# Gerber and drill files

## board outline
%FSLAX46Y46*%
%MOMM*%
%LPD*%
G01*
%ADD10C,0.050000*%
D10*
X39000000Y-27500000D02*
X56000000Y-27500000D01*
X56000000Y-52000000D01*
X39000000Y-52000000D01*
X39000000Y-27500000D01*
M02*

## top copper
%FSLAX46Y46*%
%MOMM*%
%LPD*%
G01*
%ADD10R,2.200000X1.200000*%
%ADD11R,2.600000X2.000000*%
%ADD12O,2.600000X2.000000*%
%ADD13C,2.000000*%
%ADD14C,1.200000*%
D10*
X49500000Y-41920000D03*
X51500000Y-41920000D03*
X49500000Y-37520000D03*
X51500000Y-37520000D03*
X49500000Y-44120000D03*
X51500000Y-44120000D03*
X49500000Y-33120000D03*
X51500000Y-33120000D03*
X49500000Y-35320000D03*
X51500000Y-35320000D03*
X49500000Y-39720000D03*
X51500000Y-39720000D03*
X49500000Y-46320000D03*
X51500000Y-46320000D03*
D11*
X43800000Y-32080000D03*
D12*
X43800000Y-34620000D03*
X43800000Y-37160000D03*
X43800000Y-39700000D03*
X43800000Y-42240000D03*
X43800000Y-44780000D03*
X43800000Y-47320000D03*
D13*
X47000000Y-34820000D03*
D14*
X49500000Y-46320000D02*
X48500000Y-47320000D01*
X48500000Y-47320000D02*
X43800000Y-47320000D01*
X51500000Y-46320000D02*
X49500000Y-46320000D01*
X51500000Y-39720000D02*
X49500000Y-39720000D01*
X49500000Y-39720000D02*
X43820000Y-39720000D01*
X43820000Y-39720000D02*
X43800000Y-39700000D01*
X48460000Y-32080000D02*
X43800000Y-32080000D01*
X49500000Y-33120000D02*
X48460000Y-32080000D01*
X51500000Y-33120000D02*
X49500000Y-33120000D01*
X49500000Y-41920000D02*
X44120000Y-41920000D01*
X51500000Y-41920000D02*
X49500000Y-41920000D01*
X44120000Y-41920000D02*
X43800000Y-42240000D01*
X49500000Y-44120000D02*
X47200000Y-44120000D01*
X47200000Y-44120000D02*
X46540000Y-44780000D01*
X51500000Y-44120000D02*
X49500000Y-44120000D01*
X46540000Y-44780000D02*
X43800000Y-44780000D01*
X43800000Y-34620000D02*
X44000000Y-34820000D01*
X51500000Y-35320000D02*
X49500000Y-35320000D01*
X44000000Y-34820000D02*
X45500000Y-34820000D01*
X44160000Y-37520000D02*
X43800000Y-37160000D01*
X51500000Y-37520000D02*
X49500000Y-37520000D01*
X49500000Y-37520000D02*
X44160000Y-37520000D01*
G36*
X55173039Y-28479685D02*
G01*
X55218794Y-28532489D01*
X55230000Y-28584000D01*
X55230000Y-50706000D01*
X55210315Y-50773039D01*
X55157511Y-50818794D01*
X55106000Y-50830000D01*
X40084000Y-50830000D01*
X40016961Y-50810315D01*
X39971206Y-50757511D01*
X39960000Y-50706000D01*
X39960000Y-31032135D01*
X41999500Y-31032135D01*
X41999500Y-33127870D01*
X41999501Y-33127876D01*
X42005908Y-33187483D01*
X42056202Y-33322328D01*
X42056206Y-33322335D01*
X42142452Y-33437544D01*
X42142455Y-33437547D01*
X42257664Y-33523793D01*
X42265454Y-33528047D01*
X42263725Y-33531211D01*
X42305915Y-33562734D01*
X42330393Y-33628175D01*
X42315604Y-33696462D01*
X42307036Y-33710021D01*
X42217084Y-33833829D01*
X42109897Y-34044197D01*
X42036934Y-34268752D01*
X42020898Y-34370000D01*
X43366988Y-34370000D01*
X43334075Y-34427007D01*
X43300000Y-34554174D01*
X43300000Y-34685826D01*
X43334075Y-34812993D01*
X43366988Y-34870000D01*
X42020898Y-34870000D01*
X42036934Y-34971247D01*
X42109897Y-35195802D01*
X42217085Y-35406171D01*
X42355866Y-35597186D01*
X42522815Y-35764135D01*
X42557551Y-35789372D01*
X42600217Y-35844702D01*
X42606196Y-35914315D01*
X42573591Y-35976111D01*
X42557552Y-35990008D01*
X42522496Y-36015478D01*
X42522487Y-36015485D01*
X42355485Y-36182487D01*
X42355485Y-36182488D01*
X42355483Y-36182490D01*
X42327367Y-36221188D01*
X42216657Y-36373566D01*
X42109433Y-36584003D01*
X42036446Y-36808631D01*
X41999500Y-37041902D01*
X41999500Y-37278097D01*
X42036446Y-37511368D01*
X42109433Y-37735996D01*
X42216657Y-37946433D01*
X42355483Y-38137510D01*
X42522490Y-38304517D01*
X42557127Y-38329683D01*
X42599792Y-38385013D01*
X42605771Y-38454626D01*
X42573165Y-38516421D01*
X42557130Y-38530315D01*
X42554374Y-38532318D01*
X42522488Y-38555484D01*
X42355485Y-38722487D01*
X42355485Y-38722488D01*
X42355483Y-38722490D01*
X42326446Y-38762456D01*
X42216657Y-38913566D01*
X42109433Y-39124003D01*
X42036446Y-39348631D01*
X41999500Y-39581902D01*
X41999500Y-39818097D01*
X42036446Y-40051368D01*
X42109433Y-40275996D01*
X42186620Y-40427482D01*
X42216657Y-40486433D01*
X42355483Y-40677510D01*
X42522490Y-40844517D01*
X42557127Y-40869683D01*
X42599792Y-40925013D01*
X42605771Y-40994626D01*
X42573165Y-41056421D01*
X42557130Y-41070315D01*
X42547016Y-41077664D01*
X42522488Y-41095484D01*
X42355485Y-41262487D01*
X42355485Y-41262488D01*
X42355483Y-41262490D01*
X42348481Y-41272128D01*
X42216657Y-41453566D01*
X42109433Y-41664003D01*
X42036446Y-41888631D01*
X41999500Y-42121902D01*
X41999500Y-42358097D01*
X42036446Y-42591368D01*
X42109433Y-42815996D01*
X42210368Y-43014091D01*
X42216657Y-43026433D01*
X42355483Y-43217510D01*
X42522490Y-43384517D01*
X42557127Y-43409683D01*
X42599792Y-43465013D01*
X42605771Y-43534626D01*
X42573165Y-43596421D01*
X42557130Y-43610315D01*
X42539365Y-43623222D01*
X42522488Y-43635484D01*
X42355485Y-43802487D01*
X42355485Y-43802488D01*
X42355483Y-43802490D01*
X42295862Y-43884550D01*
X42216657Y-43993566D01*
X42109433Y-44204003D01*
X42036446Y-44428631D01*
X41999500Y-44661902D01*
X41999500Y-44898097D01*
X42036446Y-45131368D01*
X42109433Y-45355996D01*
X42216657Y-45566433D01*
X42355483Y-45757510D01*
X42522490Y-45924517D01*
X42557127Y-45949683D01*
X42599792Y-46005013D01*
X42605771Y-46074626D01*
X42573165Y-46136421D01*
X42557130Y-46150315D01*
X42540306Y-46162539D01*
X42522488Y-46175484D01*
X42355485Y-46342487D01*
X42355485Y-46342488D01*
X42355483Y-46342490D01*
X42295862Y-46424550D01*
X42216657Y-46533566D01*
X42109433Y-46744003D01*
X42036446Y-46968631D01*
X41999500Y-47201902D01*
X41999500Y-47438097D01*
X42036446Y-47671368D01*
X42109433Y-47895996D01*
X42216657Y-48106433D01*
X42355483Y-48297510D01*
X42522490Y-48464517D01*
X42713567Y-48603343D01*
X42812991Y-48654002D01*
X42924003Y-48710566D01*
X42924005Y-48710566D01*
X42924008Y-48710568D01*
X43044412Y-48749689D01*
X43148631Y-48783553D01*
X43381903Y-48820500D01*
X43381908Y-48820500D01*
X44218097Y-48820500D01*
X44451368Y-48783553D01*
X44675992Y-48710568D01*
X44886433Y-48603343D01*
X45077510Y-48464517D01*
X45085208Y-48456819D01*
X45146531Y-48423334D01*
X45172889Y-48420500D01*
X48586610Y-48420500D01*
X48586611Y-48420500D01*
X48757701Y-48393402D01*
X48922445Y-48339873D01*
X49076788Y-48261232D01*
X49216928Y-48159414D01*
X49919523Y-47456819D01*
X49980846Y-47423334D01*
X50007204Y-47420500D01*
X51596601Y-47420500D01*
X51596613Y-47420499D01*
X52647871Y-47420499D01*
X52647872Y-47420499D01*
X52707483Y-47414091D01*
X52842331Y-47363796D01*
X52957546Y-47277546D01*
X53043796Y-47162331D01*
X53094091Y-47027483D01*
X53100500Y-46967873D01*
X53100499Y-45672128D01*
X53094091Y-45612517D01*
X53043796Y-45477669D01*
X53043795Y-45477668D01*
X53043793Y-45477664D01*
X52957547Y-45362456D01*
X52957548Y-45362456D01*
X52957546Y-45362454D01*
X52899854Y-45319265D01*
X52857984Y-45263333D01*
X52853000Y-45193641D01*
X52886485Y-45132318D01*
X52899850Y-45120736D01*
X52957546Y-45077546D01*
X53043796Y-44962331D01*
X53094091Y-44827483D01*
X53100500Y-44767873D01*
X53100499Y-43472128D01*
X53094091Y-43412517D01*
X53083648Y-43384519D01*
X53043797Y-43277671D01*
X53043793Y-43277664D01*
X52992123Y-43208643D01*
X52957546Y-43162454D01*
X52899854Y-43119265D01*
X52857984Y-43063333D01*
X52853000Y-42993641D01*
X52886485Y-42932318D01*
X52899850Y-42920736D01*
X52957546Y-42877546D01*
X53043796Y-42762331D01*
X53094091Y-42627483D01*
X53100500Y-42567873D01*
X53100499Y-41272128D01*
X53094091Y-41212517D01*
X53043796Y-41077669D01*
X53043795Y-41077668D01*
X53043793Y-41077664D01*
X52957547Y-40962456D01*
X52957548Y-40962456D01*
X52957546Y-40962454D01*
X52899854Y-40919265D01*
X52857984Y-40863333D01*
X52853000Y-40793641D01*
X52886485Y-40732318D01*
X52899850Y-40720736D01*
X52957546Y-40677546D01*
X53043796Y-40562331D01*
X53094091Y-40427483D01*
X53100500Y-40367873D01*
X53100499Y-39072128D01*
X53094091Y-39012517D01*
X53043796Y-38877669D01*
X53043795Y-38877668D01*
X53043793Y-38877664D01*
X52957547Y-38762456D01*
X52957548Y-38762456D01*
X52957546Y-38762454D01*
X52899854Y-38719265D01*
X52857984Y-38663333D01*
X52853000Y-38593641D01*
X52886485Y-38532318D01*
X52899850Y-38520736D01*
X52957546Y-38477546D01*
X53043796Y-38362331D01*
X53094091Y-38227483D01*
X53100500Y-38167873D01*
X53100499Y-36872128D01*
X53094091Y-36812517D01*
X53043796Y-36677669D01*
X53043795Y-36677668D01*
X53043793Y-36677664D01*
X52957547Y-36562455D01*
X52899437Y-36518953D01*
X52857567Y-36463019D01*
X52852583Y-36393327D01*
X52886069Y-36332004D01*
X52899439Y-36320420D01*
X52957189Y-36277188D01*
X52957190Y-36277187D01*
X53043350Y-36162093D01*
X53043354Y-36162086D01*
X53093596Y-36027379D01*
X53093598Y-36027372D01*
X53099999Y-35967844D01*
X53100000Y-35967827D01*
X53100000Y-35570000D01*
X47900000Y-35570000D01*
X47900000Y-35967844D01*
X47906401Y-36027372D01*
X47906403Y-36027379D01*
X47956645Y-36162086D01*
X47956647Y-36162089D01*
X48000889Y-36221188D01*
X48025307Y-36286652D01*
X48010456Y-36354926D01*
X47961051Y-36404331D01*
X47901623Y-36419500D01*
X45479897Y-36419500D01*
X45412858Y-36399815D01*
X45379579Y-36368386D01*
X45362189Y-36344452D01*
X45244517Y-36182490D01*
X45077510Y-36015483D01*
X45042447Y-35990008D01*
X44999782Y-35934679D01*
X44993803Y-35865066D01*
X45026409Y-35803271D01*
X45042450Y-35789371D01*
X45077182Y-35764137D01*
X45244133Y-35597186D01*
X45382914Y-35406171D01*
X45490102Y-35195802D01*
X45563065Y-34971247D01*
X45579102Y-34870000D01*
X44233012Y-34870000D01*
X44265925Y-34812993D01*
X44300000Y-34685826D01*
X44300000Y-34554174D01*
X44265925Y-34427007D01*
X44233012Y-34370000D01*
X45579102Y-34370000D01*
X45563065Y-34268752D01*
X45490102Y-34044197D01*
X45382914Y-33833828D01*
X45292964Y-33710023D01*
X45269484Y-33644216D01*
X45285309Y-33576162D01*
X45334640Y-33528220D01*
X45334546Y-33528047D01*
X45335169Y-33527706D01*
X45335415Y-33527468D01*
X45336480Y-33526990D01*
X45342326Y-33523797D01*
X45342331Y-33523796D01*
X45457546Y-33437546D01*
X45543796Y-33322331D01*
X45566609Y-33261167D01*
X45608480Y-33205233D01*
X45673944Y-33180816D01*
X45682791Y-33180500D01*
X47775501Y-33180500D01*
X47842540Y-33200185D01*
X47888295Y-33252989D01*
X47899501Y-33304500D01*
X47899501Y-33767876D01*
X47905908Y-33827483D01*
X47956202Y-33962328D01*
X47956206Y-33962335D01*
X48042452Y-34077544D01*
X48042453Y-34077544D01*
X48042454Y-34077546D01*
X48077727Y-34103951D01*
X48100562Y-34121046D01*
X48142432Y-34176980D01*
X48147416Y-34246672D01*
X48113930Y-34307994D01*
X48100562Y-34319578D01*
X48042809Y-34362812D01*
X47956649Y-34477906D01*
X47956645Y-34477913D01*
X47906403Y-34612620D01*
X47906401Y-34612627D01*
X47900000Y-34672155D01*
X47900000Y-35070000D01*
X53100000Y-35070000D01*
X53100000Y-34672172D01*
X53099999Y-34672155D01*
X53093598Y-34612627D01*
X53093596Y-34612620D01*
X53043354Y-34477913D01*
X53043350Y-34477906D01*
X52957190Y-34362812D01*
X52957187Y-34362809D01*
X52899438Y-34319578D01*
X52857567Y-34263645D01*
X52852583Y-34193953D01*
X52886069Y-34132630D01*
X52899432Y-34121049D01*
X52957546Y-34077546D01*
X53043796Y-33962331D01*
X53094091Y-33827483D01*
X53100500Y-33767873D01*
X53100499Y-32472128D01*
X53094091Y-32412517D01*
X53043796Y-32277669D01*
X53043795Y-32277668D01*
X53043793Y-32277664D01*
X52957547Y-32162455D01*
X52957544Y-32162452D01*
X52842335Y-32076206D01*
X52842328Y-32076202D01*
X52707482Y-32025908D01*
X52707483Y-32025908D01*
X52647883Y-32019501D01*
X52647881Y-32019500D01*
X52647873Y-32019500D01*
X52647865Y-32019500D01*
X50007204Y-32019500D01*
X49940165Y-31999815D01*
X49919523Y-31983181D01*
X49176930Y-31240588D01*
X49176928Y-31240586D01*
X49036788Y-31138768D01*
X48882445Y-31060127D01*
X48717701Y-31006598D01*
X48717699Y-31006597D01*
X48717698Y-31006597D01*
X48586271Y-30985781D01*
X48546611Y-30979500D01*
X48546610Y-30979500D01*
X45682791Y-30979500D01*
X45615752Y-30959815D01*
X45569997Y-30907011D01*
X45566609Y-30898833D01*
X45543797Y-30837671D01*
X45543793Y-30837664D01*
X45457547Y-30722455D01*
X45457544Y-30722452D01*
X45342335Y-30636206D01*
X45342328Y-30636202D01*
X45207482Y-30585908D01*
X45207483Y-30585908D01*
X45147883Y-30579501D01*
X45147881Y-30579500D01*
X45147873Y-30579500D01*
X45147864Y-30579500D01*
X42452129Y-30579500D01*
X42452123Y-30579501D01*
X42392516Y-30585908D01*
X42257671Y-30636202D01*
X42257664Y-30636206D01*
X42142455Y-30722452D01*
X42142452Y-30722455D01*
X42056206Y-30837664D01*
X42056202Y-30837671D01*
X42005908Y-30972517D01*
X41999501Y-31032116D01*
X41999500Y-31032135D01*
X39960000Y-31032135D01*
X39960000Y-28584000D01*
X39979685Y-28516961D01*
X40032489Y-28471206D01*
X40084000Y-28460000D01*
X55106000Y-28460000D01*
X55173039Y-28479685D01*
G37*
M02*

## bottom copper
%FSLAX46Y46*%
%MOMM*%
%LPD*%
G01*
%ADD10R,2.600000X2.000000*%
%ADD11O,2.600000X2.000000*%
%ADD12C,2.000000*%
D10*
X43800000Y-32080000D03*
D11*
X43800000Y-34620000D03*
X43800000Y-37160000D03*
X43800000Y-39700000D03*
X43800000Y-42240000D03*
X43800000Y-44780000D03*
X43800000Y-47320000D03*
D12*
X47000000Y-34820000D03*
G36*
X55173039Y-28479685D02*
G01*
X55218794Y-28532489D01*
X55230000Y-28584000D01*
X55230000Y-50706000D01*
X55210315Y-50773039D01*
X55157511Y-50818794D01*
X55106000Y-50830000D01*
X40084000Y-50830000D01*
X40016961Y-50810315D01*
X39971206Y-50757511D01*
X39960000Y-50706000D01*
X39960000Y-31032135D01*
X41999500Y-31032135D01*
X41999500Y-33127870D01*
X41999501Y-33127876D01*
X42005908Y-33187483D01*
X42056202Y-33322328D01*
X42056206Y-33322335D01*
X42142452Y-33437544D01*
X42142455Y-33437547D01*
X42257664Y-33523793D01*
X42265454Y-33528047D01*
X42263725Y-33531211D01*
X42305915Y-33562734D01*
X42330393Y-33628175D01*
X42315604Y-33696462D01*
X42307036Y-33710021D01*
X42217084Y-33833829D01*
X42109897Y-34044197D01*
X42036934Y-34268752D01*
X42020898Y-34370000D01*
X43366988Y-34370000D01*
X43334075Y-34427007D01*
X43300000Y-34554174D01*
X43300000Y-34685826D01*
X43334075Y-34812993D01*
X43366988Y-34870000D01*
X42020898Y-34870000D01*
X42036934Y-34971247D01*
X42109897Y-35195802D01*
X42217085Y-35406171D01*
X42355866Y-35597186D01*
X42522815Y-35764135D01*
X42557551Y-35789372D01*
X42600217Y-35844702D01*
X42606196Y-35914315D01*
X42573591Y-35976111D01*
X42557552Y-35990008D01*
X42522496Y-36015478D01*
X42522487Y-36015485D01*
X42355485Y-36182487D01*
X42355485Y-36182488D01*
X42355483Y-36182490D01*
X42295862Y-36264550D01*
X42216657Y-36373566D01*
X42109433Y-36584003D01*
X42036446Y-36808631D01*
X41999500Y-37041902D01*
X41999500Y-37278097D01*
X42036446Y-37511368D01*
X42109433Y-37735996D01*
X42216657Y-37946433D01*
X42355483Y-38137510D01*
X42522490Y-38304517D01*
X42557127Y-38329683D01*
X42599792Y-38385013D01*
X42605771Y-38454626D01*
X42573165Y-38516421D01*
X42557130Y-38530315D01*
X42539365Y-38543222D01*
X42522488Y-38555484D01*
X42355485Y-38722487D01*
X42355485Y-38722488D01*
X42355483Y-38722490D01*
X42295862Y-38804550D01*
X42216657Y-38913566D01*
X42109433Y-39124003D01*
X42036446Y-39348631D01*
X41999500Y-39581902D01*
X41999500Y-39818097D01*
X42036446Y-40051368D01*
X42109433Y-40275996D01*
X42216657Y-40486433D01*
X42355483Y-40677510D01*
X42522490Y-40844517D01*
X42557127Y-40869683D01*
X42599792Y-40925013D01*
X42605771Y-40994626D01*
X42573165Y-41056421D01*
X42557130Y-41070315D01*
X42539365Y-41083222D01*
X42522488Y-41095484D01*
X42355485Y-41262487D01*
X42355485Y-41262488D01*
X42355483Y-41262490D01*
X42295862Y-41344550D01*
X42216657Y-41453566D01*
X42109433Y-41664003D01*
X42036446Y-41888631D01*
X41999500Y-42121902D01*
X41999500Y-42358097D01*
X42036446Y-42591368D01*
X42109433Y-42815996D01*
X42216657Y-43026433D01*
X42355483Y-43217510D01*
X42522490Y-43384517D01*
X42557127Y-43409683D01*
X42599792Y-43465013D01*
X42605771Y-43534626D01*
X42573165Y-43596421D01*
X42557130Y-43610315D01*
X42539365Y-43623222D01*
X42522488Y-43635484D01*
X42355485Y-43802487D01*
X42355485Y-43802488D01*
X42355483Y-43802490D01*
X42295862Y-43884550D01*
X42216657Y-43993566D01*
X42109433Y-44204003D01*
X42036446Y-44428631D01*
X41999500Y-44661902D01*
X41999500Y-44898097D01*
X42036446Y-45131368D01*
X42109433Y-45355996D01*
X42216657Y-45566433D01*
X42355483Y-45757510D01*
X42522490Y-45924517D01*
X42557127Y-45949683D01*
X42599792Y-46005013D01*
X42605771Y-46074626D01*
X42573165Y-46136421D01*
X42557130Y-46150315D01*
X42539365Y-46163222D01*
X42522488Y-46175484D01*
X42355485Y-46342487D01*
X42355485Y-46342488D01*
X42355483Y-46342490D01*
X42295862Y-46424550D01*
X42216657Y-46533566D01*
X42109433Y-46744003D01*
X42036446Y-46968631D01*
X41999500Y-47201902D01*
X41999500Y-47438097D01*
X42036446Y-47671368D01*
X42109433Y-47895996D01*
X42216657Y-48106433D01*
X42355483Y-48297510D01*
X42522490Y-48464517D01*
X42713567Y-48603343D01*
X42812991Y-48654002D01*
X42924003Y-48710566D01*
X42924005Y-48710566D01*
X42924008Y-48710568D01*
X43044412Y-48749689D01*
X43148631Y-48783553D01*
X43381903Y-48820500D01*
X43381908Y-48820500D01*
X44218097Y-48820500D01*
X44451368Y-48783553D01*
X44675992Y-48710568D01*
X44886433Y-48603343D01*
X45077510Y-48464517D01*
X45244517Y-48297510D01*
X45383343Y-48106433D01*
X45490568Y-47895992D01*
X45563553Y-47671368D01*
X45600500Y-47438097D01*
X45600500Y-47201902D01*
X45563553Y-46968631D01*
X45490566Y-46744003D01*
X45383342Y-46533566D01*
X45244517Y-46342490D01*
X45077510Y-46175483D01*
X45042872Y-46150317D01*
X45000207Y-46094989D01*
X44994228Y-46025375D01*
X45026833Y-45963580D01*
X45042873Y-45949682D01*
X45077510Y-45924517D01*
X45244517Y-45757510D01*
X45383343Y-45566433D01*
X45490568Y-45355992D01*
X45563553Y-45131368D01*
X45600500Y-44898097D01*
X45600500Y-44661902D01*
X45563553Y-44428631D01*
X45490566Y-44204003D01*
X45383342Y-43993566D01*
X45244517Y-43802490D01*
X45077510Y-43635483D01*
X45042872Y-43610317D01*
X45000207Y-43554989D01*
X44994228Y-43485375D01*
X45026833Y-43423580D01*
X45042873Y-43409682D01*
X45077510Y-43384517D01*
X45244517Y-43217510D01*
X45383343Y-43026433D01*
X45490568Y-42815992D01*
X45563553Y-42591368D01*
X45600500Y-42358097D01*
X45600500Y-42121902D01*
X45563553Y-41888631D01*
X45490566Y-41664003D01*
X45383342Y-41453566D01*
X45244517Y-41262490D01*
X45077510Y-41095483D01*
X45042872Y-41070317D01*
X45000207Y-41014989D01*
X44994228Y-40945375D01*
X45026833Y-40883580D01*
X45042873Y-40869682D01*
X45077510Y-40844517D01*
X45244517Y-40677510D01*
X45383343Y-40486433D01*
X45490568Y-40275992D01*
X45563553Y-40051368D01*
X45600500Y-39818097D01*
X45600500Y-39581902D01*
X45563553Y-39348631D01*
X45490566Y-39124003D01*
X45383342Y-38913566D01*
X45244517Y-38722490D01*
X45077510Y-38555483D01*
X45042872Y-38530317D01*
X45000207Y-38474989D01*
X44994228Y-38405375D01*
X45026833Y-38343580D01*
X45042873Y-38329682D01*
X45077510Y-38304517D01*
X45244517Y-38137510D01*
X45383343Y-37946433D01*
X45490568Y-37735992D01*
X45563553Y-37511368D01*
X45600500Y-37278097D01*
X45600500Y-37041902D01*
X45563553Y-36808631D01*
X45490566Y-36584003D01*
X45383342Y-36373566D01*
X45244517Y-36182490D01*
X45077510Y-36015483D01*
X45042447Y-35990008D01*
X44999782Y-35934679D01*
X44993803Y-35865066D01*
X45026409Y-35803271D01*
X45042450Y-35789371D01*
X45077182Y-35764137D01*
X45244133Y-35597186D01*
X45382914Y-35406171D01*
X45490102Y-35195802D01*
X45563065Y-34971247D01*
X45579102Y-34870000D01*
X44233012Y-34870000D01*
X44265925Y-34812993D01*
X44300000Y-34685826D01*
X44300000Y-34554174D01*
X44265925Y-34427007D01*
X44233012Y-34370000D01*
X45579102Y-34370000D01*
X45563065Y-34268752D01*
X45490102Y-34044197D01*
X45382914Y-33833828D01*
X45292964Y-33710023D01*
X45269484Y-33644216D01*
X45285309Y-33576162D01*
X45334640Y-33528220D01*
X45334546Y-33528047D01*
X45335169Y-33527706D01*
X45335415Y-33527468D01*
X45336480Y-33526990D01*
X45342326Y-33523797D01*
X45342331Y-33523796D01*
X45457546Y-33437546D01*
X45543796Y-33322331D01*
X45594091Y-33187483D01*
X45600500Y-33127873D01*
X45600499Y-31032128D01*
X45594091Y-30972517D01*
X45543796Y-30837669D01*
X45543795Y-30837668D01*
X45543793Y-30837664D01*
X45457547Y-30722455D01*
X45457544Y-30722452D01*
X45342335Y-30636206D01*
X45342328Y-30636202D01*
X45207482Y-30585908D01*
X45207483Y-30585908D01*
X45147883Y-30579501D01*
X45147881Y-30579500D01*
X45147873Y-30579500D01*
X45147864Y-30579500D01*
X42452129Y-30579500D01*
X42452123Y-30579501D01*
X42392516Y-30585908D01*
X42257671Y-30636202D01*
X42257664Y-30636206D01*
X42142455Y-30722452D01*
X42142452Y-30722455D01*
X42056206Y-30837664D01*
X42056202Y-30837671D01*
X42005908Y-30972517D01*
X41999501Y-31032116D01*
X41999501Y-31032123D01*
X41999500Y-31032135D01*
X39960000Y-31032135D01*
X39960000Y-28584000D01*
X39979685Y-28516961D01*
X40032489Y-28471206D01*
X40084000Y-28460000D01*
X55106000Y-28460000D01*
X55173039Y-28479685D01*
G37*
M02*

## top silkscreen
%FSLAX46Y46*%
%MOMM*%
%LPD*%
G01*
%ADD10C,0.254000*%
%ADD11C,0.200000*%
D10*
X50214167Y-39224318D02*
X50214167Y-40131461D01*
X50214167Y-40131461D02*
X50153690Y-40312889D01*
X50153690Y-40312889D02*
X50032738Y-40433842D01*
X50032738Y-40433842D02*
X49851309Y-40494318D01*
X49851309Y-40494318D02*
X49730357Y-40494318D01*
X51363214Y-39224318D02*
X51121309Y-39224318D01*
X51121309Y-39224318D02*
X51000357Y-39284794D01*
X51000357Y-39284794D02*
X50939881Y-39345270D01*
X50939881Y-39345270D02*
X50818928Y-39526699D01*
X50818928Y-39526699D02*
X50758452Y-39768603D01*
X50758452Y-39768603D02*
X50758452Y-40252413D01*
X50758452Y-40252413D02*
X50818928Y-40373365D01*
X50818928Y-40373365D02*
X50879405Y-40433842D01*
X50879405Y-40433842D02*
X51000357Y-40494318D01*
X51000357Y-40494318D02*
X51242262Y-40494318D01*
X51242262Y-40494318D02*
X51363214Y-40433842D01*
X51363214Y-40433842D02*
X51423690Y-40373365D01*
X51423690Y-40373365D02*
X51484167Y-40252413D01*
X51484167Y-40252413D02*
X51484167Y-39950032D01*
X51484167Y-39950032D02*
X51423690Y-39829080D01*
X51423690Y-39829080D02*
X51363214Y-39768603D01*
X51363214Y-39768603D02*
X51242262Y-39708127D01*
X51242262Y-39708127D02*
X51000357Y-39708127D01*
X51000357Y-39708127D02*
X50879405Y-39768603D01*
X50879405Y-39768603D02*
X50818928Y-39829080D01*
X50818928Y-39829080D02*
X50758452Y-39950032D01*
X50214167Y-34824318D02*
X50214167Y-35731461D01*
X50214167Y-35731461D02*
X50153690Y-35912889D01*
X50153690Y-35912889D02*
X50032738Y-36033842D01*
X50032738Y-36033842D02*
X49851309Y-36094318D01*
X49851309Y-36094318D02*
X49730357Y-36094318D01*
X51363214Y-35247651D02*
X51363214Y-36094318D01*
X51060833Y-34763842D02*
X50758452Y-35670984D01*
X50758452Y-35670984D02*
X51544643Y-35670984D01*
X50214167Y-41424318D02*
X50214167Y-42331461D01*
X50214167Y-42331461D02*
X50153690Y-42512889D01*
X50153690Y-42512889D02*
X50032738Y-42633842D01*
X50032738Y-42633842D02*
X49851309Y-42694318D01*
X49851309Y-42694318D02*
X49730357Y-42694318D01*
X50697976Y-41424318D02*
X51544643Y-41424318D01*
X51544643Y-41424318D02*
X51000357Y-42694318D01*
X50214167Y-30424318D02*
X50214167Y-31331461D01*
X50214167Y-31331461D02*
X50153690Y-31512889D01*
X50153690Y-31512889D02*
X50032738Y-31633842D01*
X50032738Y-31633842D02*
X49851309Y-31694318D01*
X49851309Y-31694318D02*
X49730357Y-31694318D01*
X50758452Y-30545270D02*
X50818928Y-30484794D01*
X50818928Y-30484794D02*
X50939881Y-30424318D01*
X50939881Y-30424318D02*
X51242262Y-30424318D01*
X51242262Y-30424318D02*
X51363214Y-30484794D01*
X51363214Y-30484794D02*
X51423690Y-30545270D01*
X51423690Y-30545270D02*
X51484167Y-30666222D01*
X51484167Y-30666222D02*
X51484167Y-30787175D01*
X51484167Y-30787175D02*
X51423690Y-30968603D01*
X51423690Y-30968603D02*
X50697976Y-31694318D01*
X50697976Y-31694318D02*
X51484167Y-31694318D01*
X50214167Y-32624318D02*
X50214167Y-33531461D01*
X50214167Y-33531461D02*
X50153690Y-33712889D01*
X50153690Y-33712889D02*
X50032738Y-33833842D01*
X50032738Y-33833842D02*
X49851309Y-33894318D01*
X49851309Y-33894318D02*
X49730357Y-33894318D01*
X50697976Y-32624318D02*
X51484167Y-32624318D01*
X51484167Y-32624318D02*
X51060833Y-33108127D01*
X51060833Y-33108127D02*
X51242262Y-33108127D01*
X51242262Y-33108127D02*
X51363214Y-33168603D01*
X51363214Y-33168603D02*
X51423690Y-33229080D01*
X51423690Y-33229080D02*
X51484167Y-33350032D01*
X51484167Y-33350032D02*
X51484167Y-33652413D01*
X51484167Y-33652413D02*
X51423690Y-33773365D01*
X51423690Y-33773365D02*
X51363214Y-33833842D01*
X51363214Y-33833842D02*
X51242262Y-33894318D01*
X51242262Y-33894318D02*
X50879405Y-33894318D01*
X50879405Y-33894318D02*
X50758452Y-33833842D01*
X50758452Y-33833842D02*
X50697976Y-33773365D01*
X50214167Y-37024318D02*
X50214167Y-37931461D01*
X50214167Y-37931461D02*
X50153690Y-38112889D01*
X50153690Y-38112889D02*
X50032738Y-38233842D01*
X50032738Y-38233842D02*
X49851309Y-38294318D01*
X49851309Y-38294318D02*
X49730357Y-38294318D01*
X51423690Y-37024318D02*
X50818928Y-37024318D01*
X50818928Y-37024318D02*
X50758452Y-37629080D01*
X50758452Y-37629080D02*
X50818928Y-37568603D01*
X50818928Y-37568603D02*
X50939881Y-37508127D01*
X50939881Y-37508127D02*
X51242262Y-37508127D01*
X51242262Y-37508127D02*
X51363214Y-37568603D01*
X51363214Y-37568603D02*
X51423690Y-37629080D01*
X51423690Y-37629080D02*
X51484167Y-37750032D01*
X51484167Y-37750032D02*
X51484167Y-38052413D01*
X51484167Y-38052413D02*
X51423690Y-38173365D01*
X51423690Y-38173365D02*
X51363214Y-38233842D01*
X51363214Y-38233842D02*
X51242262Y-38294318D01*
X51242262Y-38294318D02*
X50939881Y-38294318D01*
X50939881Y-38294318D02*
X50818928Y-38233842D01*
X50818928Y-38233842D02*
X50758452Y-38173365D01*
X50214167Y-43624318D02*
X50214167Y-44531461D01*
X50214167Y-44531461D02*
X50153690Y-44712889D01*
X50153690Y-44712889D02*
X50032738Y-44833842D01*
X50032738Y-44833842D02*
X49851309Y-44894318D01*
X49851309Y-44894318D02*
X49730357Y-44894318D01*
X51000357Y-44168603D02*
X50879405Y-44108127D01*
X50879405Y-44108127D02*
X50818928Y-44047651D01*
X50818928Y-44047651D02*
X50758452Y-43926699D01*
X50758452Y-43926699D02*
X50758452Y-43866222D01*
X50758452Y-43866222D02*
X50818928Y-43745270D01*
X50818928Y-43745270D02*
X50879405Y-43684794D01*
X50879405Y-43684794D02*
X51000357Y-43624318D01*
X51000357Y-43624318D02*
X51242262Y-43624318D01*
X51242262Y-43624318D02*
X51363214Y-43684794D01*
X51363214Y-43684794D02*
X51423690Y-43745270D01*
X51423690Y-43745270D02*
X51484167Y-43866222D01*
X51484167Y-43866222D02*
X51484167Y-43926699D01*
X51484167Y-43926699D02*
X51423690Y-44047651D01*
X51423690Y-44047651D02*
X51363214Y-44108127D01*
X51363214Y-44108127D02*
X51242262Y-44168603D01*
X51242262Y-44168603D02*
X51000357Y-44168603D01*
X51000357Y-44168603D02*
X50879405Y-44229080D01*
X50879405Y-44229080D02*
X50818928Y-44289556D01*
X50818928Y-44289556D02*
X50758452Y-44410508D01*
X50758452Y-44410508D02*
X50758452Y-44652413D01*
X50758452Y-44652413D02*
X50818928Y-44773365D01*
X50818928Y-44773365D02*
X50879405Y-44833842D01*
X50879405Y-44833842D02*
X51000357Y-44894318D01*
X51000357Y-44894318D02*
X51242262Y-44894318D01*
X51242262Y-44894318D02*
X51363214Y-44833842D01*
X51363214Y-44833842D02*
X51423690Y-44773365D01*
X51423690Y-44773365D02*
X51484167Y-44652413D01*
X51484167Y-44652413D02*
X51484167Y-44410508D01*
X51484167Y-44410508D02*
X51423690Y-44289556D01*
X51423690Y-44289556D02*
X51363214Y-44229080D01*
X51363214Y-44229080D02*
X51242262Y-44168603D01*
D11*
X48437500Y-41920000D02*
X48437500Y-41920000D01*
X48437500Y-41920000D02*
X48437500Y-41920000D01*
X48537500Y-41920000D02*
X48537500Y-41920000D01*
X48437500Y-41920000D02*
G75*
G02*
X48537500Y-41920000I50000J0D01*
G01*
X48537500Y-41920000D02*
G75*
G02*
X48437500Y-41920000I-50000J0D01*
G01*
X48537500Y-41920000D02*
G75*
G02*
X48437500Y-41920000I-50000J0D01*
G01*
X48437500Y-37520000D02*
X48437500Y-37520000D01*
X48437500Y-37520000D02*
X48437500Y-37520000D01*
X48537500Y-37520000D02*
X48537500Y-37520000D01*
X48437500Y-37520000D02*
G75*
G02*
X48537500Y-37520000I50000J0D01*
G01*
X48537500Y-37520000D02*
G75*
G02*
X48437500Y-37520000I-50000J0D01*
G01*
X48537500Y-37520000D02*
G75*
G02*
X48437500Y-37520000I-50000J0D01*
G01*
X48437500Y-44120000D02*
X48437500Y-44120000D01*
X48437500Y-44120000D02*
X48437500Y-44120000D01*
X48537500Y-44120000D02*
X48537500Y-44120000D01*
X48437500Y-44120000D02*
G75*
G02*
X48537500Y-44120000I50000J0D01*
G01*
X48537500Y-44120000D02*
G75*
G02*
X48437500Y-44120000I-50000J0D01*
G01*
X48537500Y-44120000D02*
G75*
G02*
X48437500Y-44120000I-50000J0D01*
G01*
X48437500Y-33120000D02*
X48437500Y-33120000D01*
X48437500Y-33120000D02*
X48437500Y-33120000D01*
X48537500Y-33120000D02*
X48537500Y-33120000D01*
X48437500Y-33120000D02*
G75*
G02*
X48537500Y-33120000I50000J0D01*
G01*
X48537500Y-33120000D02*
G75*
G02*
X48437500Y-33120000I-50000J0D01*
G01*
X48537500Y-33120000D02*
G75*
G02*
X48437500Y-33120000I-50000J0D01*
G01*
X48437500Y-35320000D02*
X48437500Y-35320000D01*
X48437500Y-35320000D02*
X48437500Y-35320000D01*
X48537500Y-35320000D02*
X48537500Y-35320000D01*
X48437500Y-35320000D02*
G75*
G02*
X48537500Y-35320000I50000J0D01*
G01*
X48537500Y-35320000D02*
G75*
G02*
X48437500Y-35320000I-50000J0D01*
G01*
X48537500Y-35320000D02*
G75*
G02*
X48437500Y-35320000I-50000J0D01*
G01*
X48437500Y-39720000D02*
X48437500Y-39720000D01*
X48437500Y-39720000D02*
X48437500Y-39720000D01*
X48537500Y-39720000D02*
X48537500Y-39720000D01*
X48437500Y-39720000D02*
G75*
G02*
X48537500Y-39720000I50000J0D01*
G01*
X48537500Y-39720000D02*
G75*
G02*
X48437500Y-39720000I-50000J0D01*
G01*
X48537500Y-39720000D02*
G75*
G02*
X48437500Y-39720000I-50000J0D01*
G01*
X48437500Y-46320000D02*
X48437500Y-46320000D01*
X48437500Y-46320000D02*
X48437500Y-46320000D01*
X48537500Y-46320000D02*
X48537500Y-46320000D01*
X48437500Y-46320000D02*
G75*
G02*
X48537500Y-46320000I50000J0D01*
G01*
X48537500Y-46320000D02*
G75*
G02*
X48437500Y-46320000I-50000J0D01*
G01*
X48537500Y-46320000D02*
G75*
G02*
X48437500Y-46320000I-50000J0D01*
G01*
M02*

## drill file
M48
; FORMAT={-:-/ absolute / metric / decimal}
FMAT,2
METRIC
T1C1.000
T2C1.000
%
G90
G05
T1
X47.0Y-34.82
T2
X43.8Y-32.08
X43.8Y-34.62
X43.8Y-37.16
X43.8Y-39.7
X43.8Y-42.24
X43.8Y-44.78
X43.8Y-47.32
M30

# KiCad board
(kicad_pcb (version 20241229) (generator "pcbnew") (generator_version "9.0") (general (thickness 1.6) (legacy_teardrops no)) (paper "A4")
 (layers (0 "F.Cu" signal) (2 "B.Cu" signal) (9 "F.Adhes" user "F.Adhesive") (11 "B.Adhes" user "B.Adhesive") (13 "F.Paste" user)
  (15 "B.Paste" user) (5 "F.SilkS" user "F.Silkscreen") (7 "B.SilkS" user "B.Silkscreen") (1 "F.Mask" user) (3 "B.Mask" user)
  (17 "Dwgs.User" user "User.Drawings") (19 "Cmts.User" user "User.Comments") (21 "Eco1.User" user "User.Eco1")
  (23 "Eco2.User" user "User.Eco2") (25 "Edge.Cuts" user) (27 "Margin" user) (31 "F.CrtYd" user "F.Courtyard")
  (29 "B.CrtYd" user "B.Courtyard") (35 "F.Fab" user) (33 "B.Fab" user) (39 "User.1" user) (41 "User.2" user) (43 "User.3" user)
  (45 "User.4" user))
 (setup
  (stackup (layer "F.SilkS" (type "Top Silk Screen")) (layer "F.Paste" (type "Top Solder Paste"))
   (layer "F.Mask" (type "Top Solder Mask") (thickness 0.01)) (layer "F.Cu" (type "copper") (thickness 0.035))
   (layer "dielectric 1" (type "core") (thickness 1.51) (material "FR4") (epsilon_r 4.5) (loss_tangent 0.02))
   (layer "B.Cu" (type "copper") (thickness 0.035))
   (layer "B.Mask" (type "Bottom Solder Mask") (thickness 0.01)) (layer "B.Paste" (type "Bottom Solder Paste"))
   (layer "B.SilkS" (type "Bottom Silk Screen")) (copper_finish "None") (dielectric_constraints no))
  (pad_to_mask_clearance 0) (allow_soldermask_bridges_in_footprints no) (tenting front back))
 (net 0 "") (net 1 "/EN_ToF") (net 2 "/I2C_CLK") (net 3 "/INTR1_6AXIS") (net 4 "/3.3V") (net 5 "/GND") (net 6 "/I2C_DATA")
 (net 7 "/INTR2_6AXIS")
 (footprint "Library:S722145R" (layer "F.Cu") (at 50.6375 41.92)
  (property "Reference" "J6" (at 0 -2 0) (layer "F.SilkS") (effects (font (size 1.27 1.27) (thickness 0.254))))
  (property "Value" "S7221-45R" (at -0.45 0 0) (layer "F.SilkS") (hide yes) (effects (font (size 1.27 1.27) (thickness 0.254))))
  (fp_line (start -2.2 0) (end -2.2 0) (stroke (width 0.2) (type solid)) (layer "F.SilkS"))
  (fp_line (start -2.2 0) (end -2.2 0) (stroke (width 0.2) (type solid)) (layer "F.SilkS"))
  (fp_line (start -2.1 0) (end -2.1 0) (stroke (width 0.2) (type solid)) (layer "F.SilkS"))
  (fp_arc (start -2.2 0) (mid -2.15 -0.05) (end -2.1 0) (stroke (width 0.2) (type solid)) (layer "F.SilkS"))
  (fp_arc (start -2.1 0) (mid -2.15 0.05) (end -2.2 0) (stroke (width 0.2) (type solid)) (layer "F.SilkS"))
  (fp_arc (start -2.1 0) (mid -2.15 0.05) (end -2.2 0) (stroke (width 0.2) (type solid)) (layer "F.SilkS"))
  (pad "1" smd rect (at -1.1375 0) (size 2.2 1.2) (layers "F.Cu" "F.Mask" "F.Paste") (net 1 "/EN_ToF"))
  (pad "2" smd rect (at 0.8625 0) (size 2.2 1.2) (layers "F.Cu" "F.Mask" "F.Paste") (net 1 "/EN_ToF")))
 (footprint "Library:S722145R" (layer "F.Cu") (at 50.6375 37.52)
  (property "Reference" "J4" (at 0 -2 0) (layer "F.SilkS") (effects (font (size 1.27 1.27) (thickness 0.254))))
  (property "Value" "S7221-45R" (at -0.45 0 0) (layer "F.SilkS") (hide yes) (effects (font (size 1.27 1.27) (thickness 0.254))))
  (fp_line (start -2.2 0) (end -2.2 0) (stroke (width 0.2) (type solid)) (layer "F.SilkS"))
  (fp_line (start -2.2 0) (end -2.2 0) (stroke (width 0.2) (type solid)) (layer "F.SilkS"))
  (fp_line (start -2.1 0) (end -2.1 0) (stroke (width 0.2) (type solid)) (layer "F.SilkS"))
  (fp_arc (start -2.2 0) (mid -2.15 -0.05) (end -2.1 0) (stroke (width 0.2) (type solid)) (layer "F.SilkS"))
  (fp_arc (start -2.1 0) (mid -2.15 0.05) (end -2.2 0) (stroke (width 0.2) (type solid)) (layer "F.SilkS"))
  (fp_arc (start -2.1 0) (mid -2.15 0.05) (end -2.2 0) (stroke (width 0.2) (type solid)) (layer "F.SilkS"))
  (pad "1" smd rect (at -1.1375 0) (size 2.2 1.2) (layers "F.Cu" "F.Mask" "F.Paste") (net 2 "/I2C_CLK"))
  (pad "2" smd rect (at 0.8625 0) (size 2.2 1.2) (layers "F.Cu" "F.Mask" "F.Paste") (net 2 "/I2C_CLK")))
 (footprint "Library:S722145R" (layer "F.Cu") (at 50.6375 44.12)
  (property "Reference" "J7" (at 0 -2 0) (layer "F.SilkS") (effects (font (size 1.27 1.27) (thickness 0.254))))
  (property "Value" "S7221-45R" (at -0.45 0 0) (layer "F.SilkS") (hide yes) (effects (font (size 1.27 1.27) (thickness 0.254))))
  (fp_line (start -2.2 0) (end -2.2 0) (stroke (width 0.2) (type solid)) (layer "F.SilkS"))
  (fp_line (start -2.2 0) (end -2.2 0) (stroke (width 0.2) (type solid)) (layer "F.SilkS"))
  (fp_line (start -2.1 0) (end -2.1 0) (stroke (width 0.2) (type solid)) (layer "F.SilkS"))
  (fp_arc (start -2.2 0) (mid -2.15 -0.05) (end -2.1 0) (stroke (width 0.2) (type solid)) (layer "F.SilkS"))
  (fp_arc (start -2.1 0) (mid -2.15 0.05) (end -2.2 0) (stroke (width 0.2) (type solid)) (layer "F.SilkS"))
  (fp_arc (start -2.1 0) (mid -2.15 0.05) (end -2.2 0) (stroke (width 0.2) (type solid)) (layer "F.SilkS"))
  (pad "1" smd rect (at -1.1375 0) (size 2.2 1.2) (layers "F.Cu" "F.Mask" "F.Paste") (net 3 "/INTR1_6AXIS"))
  (pad "2" smd rect (at 0.8625 0) (size 2.2 1.2) (layers "F.Cu" "F.Mask" "F.Paste") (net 3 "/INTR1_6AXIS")))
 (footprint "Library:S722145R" (layer "F.Cu") (at 50.6375 33.12)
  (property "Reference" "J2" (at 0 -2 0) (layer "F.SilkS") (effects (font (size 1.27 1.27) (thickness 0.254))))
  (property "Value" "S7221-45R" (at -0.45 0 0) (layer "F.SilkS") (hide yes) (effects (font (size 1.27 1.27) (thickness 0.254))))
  (fp_line (start -2.2 0) (end -2.2 0) (stroke (width 0.2) (type solid)) (layer "F.SilkS"))
  (fp_line (start -2.2 0) (end -2.2 0) (stroke (width 0.2) (type solid)) (layer "F.SilkS"))
  (fp_line (start -2.1 0) (end -2.1 0) (stroke (width 0.2) (type solid)) (layer "F.SilkS"))
  (fp_arc (start -2.2 0) (mid -2.15 -0.05) (end -2.1 0) (stroke (width 0.2) (type solid)) (layer "F.SilkS"))
  (fp_arc (start -2.1 0) (mid -2.15 0.05) (end -2.2 0) (stroke (width 0.2) (type solid)) (layer "F.SilkS"))
  (fp_arc (start -2.1 0) (mid -2.15 0.05) (end -2.2 0) (stroke (width 0.2) (type solid)) (layer "F.SilkS"))
  (pad "1" smd rect (at -1.1375 0) (size 2.2 1.2) (layers "F.Cu" "F.Mask" "F.Paste") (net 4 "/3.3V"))
  (pad "2" smd rect (at 0.8625 0) (size 2.2 1.2) (layers "F.Cu" "F.Mask" "F.Paste") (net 4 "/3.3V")))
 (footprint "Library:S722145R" (layer "F.Cu") (at 50.6375 35.32)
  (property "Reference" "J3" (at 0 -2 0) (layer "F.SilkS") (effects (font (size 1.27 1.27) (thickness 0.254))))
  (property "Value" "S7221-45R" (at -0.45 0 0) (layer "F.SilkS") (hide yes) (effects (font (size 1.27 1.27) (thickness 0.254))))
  (fp_line (start -2.2 0) (end -2.2 0) (stroke (width 0.2) (type solid)) (layer "F.SilkS"))
  (fp_line (start -2.2 0) (end -2.2 0) (stroke (width 0.2) (type solid)) (layer "F.SilkS"))
  (fp_line (start -2.1 0) (end -2.1 0) (stroke (width 0.2) (type solid)) (layer "F.SilkS"))
  (fp_arc (start -2.2 0) (mid -2.15 -0.05) (end -2.1 0) (stroke (width 0.2) (type solid)) (layer "F.SilkS"))
  (fp_arc (start -2.1 0) (mid -2.15 0.05) (end -2.2 0) (stroke (width 0.2) (type solid)) (layer "F.SilkS"))
  (fp_arc (start -2.1 0) (mid -2.15 0.05) (end -2.2 0) (stroke (width 0.2) (type solid)) (layer "F.SilkS"))
  (pad "1" smd rect (at -1.1375 0) (size 2.2 1.2) (layers "F.Cu" "F.Mask" "F.Paste") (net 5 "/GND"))
  (pad "2" smd rect (at 0.8625 0) (size 2.2 1.2) (layers "F.Cu" "F.Mask" "F.Paste") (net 5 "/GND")))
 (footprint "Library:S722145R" (layer "F.Cu") (at 50.6375 39.72)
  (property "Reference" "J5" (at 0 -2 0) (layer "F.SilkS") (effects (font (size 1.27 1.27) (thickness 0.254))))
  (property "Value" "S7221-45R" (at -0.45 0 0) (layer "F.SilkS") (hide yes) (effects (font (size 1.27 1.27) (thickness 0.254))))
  (fp_line (start -2.2 0) (end -2.2 0) (stroke (width 0.2) (type solid)) (layer "F.SilkS"))
  (fp_line (start -2.2 0) (end -2.2 0) (stroke (width 0.2) (type solid)) (layer "F.SilkS"))
  (fp_line (start -2.1 0) (end -2.1 0) (stroke (width 0.2) (type solid)) (layer "F.SilkS"))
  (fp_arc (start -2.2 0) (mid -2.15 -0.05) (end -2.1 0) (stroke (width 0.2) (type solid)) (layer "F.SilkS"))
  (fp_arc (start -2.1 0) (mid -2.15 0.05) (end -2.2 0) (stroke (width 0.2) (type solid)) (layer "F.SilkS"))
  (fp_arc (start -2.1 0) (mid -2.15 0.05) (end -2.2 0) (stroke (width 0.2) (type solid)) (layer "F.SilkS"))
  (pad "1" smd rect (at -1.1375 0) (size 2.2 1.2) (layers "F.Cu" "F.Mask" "F.Paste") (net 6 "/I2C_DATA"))
  (pad "2" smd rect (at 0.8625 0) (size 2.2 1.2) (layers "F.Cu" "F.Mask" "F.Paste") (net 6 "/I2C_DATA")))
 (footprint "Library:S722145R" (layer "F.Cu") (at 50.6375 46.32)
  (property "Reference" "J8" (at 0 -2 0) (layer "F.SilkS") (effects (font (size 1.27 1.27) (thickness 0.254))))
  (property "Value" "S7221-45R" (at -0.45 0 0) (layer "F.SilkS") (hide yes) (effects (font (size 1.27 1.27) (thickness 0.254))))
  (fp_line (start -2.2 0) (end -2.2 0) (stroke (width 0.2) (type solid)) (layer "F.SilkS"))
  (fp_line (start -2.2 0) (end -2.2 0) (stroke (width 0.2) (type solid)) (layer "F.SilkS"))
  (fp_line (start -2.1 0) (end -2.1 0) (stroke (width 0.2) (type solid)) (layer "F.SilkS"))
  (fp_arc (start -2.2 0) (mid -2.15 -0.05) (end -2.1 0) (stroke (width 0.2) (type solid)) (layer "F.SilkS"))
  (fp_arc (start -2.1 0) (mid -2.15 0.05) (end -2.2 0) (stroke (width 0.2) (type solid)) (layer "F.SilkS"))
  (fp_arc (start -2.1 0) (mid -2.15 0.05) (end -2.2 0) (stroke (width 0.2) (type solid)) (layer "F.SilkS"))
  (pad "1" smd rect (at -1.1375 0) (size 2.2 1.2) (layers "F.Cu" "F.Mask" "F.Paste") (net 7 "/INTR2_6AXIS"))
  (pad "2" smd rect (at 0.8625 0) (size 2.2 1.2) (layers "F.Cu" "F.Mask" "F.Paste") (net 7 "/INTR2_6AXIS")))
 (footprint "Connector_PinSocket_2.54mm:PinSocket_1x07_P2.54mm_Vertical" (layer "B.Cu") (at 43.8 32.08 180)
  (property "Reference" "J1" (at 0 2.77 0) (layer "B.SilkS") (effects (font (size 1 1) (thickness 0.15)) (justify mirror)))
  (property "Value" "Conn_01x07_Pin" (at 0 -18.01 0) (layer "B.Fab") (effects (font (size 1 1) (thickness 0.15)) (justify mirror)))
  (pad "1" thru_hole rect (at 0 0 180) (size 2.6 2) (drill 1) (layers "*.Cu" "*.Mask") (remove_unused_layers no) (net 4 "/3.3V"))
  (pad "2" thru_hole oval (at 0 -2.54 180) (size 2.6 2) (drill 1) (layers "*.Cu" "*.Mask") (remove_unused_layers no) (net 5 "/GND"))
  (pad "3" thru_hole oval (at 0 -5.08 180) (size 2.6 2) (drill 1) (layers "*.Cu" "*.Mask") (remove_unused_layers no) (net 2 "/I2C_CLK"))
  (pad "4" thru_hole oval (at 0 -7.62 180) (size 2.6 2) (drill 1) (layers "*.Cu" "*.Mask") (remove_unused_layers no) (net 6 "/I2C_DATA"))
  (pad "5" thru_hole oval (at 0 -10.16 180) (size 2.6 2) (drill 1) (layers "*.Cu" "*.Mask") (remove_unused_layers no) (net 1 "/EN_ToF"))
  (pad "6" thru_hole oval (at 0 -12.7 180) (size 2.6 2) (drill 1) (layers "*.Cu" "*.Mask") (remove_unused_layers no) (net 3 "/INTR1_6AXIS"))
  (pad "7" thru_hole oval (at 0 -15.24 180) (size 2.6 2) (drill 1) (layers "*.Cu" "*.Mask") (remove_unused_layers no) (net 7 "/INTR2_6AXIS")))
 (gr_rect (start 39 27.5) (end 56 52) (stroke (width 0.05) (type solid)) (fill no) (layer "Edge.Cuts"))
 (segment (start 49.5 46.32) (end 48.5 47.32) (width 1.2) (layer "F.Cu") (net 7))
 (segment (start 48.5 47.32) (end 43.8 47.32) (width 1.2) (layer "F.Cu") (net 7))
 (segment (start 51.5 46.32) (end 49.5 46.32) (width 1.2) (layer "F.Cu") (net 7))
 (segment (start 51.5 39.72) (end 49.5 39.72) (width 1.2) (layer "F.Cu") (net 6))
 (segment (start 49.5 39.72) (end 43.82 39.72) (width 1.2) (layer "F.Cu") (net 6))
 (segment (start 43.82 39.72) (end 43.8 39.7) (width 1.2) (layer "F.Cu") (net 6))
 (segment (start 48.46 32.08) (end 43.8 32.08) (width 1.2) (layer "F.Cu") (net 4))
 (segment (start 49.5 33.12) (end 48.46 32.08) (width 1.2) (layer "F.Cu") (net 4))
 (segment (start 51.5 33.12) (end 49.5 33.12) (width 1.2) (layer "F.Cu") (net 4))
 (segment (start 49.5 41.92) (end 44.12 41.92) (width 1.2) (layer "F.Cu") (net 1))
 (segment (start 51.5 41.92) (end 49.5 41.92) (width 1.2) (layer "F.Cu") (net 1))
 (segment (start 44.12 41.92) (end 43.8 42.24) (width 1.2) (layer "F.Cu") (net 1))
 (segment (start 49.5 44.12) (end 47.2 44.12) (width 1.2) (layer "F.Cu") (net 3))
 (segment (start 47.2 44.12) (end 46.54 44.78) (width 1.2) (layer "F.Cu") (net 3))
 (segment (start 51.5 44.12) (end 49.5 44.12) (width 1.2) (layer "F.Cu") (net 3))
 (segment (start 46.54 44.78) (end 43.8 44.78) (width 1.2) (layer "F.Cu") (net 3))
 (segment (start 43.8 34.62) (end 44 34.82) (width 1.2) (layer "F.Cu") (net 5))
 (segment (start 51.5 35.32) (end 49.5 35.32) (width 1.2) (layer "F.Cu") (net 5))
 (segment (start 44 34.82) (end 45.5 34.82) (width 1.2) (layer "F.Cu") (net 5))
 (via (at 47 34.82) (size 2) (drill 1) (layers "F.Cu" "B.Cu") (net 5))
 (segment (start 44.16 37.52) (end 43.8 37.16) (width 1.2) (layer "F.Cu") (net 2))
 (segment (start 51.5 37.52) (end 49.5 37.52) (width 1.2) (layer "F.Cu") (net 2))
 (segment (start 49.5 37.52) (end 44.16 37.52) (width 1.2) (layer "F.Cu") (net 2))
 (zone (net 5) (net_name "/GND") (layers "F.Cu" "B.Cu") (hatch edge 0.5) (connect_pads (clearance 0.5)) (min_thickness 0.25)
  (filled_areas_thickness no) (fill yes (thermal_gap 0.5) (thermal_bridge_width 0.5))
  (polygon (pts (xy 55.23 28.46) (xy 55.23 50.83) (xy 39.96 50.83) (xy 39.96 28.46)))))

